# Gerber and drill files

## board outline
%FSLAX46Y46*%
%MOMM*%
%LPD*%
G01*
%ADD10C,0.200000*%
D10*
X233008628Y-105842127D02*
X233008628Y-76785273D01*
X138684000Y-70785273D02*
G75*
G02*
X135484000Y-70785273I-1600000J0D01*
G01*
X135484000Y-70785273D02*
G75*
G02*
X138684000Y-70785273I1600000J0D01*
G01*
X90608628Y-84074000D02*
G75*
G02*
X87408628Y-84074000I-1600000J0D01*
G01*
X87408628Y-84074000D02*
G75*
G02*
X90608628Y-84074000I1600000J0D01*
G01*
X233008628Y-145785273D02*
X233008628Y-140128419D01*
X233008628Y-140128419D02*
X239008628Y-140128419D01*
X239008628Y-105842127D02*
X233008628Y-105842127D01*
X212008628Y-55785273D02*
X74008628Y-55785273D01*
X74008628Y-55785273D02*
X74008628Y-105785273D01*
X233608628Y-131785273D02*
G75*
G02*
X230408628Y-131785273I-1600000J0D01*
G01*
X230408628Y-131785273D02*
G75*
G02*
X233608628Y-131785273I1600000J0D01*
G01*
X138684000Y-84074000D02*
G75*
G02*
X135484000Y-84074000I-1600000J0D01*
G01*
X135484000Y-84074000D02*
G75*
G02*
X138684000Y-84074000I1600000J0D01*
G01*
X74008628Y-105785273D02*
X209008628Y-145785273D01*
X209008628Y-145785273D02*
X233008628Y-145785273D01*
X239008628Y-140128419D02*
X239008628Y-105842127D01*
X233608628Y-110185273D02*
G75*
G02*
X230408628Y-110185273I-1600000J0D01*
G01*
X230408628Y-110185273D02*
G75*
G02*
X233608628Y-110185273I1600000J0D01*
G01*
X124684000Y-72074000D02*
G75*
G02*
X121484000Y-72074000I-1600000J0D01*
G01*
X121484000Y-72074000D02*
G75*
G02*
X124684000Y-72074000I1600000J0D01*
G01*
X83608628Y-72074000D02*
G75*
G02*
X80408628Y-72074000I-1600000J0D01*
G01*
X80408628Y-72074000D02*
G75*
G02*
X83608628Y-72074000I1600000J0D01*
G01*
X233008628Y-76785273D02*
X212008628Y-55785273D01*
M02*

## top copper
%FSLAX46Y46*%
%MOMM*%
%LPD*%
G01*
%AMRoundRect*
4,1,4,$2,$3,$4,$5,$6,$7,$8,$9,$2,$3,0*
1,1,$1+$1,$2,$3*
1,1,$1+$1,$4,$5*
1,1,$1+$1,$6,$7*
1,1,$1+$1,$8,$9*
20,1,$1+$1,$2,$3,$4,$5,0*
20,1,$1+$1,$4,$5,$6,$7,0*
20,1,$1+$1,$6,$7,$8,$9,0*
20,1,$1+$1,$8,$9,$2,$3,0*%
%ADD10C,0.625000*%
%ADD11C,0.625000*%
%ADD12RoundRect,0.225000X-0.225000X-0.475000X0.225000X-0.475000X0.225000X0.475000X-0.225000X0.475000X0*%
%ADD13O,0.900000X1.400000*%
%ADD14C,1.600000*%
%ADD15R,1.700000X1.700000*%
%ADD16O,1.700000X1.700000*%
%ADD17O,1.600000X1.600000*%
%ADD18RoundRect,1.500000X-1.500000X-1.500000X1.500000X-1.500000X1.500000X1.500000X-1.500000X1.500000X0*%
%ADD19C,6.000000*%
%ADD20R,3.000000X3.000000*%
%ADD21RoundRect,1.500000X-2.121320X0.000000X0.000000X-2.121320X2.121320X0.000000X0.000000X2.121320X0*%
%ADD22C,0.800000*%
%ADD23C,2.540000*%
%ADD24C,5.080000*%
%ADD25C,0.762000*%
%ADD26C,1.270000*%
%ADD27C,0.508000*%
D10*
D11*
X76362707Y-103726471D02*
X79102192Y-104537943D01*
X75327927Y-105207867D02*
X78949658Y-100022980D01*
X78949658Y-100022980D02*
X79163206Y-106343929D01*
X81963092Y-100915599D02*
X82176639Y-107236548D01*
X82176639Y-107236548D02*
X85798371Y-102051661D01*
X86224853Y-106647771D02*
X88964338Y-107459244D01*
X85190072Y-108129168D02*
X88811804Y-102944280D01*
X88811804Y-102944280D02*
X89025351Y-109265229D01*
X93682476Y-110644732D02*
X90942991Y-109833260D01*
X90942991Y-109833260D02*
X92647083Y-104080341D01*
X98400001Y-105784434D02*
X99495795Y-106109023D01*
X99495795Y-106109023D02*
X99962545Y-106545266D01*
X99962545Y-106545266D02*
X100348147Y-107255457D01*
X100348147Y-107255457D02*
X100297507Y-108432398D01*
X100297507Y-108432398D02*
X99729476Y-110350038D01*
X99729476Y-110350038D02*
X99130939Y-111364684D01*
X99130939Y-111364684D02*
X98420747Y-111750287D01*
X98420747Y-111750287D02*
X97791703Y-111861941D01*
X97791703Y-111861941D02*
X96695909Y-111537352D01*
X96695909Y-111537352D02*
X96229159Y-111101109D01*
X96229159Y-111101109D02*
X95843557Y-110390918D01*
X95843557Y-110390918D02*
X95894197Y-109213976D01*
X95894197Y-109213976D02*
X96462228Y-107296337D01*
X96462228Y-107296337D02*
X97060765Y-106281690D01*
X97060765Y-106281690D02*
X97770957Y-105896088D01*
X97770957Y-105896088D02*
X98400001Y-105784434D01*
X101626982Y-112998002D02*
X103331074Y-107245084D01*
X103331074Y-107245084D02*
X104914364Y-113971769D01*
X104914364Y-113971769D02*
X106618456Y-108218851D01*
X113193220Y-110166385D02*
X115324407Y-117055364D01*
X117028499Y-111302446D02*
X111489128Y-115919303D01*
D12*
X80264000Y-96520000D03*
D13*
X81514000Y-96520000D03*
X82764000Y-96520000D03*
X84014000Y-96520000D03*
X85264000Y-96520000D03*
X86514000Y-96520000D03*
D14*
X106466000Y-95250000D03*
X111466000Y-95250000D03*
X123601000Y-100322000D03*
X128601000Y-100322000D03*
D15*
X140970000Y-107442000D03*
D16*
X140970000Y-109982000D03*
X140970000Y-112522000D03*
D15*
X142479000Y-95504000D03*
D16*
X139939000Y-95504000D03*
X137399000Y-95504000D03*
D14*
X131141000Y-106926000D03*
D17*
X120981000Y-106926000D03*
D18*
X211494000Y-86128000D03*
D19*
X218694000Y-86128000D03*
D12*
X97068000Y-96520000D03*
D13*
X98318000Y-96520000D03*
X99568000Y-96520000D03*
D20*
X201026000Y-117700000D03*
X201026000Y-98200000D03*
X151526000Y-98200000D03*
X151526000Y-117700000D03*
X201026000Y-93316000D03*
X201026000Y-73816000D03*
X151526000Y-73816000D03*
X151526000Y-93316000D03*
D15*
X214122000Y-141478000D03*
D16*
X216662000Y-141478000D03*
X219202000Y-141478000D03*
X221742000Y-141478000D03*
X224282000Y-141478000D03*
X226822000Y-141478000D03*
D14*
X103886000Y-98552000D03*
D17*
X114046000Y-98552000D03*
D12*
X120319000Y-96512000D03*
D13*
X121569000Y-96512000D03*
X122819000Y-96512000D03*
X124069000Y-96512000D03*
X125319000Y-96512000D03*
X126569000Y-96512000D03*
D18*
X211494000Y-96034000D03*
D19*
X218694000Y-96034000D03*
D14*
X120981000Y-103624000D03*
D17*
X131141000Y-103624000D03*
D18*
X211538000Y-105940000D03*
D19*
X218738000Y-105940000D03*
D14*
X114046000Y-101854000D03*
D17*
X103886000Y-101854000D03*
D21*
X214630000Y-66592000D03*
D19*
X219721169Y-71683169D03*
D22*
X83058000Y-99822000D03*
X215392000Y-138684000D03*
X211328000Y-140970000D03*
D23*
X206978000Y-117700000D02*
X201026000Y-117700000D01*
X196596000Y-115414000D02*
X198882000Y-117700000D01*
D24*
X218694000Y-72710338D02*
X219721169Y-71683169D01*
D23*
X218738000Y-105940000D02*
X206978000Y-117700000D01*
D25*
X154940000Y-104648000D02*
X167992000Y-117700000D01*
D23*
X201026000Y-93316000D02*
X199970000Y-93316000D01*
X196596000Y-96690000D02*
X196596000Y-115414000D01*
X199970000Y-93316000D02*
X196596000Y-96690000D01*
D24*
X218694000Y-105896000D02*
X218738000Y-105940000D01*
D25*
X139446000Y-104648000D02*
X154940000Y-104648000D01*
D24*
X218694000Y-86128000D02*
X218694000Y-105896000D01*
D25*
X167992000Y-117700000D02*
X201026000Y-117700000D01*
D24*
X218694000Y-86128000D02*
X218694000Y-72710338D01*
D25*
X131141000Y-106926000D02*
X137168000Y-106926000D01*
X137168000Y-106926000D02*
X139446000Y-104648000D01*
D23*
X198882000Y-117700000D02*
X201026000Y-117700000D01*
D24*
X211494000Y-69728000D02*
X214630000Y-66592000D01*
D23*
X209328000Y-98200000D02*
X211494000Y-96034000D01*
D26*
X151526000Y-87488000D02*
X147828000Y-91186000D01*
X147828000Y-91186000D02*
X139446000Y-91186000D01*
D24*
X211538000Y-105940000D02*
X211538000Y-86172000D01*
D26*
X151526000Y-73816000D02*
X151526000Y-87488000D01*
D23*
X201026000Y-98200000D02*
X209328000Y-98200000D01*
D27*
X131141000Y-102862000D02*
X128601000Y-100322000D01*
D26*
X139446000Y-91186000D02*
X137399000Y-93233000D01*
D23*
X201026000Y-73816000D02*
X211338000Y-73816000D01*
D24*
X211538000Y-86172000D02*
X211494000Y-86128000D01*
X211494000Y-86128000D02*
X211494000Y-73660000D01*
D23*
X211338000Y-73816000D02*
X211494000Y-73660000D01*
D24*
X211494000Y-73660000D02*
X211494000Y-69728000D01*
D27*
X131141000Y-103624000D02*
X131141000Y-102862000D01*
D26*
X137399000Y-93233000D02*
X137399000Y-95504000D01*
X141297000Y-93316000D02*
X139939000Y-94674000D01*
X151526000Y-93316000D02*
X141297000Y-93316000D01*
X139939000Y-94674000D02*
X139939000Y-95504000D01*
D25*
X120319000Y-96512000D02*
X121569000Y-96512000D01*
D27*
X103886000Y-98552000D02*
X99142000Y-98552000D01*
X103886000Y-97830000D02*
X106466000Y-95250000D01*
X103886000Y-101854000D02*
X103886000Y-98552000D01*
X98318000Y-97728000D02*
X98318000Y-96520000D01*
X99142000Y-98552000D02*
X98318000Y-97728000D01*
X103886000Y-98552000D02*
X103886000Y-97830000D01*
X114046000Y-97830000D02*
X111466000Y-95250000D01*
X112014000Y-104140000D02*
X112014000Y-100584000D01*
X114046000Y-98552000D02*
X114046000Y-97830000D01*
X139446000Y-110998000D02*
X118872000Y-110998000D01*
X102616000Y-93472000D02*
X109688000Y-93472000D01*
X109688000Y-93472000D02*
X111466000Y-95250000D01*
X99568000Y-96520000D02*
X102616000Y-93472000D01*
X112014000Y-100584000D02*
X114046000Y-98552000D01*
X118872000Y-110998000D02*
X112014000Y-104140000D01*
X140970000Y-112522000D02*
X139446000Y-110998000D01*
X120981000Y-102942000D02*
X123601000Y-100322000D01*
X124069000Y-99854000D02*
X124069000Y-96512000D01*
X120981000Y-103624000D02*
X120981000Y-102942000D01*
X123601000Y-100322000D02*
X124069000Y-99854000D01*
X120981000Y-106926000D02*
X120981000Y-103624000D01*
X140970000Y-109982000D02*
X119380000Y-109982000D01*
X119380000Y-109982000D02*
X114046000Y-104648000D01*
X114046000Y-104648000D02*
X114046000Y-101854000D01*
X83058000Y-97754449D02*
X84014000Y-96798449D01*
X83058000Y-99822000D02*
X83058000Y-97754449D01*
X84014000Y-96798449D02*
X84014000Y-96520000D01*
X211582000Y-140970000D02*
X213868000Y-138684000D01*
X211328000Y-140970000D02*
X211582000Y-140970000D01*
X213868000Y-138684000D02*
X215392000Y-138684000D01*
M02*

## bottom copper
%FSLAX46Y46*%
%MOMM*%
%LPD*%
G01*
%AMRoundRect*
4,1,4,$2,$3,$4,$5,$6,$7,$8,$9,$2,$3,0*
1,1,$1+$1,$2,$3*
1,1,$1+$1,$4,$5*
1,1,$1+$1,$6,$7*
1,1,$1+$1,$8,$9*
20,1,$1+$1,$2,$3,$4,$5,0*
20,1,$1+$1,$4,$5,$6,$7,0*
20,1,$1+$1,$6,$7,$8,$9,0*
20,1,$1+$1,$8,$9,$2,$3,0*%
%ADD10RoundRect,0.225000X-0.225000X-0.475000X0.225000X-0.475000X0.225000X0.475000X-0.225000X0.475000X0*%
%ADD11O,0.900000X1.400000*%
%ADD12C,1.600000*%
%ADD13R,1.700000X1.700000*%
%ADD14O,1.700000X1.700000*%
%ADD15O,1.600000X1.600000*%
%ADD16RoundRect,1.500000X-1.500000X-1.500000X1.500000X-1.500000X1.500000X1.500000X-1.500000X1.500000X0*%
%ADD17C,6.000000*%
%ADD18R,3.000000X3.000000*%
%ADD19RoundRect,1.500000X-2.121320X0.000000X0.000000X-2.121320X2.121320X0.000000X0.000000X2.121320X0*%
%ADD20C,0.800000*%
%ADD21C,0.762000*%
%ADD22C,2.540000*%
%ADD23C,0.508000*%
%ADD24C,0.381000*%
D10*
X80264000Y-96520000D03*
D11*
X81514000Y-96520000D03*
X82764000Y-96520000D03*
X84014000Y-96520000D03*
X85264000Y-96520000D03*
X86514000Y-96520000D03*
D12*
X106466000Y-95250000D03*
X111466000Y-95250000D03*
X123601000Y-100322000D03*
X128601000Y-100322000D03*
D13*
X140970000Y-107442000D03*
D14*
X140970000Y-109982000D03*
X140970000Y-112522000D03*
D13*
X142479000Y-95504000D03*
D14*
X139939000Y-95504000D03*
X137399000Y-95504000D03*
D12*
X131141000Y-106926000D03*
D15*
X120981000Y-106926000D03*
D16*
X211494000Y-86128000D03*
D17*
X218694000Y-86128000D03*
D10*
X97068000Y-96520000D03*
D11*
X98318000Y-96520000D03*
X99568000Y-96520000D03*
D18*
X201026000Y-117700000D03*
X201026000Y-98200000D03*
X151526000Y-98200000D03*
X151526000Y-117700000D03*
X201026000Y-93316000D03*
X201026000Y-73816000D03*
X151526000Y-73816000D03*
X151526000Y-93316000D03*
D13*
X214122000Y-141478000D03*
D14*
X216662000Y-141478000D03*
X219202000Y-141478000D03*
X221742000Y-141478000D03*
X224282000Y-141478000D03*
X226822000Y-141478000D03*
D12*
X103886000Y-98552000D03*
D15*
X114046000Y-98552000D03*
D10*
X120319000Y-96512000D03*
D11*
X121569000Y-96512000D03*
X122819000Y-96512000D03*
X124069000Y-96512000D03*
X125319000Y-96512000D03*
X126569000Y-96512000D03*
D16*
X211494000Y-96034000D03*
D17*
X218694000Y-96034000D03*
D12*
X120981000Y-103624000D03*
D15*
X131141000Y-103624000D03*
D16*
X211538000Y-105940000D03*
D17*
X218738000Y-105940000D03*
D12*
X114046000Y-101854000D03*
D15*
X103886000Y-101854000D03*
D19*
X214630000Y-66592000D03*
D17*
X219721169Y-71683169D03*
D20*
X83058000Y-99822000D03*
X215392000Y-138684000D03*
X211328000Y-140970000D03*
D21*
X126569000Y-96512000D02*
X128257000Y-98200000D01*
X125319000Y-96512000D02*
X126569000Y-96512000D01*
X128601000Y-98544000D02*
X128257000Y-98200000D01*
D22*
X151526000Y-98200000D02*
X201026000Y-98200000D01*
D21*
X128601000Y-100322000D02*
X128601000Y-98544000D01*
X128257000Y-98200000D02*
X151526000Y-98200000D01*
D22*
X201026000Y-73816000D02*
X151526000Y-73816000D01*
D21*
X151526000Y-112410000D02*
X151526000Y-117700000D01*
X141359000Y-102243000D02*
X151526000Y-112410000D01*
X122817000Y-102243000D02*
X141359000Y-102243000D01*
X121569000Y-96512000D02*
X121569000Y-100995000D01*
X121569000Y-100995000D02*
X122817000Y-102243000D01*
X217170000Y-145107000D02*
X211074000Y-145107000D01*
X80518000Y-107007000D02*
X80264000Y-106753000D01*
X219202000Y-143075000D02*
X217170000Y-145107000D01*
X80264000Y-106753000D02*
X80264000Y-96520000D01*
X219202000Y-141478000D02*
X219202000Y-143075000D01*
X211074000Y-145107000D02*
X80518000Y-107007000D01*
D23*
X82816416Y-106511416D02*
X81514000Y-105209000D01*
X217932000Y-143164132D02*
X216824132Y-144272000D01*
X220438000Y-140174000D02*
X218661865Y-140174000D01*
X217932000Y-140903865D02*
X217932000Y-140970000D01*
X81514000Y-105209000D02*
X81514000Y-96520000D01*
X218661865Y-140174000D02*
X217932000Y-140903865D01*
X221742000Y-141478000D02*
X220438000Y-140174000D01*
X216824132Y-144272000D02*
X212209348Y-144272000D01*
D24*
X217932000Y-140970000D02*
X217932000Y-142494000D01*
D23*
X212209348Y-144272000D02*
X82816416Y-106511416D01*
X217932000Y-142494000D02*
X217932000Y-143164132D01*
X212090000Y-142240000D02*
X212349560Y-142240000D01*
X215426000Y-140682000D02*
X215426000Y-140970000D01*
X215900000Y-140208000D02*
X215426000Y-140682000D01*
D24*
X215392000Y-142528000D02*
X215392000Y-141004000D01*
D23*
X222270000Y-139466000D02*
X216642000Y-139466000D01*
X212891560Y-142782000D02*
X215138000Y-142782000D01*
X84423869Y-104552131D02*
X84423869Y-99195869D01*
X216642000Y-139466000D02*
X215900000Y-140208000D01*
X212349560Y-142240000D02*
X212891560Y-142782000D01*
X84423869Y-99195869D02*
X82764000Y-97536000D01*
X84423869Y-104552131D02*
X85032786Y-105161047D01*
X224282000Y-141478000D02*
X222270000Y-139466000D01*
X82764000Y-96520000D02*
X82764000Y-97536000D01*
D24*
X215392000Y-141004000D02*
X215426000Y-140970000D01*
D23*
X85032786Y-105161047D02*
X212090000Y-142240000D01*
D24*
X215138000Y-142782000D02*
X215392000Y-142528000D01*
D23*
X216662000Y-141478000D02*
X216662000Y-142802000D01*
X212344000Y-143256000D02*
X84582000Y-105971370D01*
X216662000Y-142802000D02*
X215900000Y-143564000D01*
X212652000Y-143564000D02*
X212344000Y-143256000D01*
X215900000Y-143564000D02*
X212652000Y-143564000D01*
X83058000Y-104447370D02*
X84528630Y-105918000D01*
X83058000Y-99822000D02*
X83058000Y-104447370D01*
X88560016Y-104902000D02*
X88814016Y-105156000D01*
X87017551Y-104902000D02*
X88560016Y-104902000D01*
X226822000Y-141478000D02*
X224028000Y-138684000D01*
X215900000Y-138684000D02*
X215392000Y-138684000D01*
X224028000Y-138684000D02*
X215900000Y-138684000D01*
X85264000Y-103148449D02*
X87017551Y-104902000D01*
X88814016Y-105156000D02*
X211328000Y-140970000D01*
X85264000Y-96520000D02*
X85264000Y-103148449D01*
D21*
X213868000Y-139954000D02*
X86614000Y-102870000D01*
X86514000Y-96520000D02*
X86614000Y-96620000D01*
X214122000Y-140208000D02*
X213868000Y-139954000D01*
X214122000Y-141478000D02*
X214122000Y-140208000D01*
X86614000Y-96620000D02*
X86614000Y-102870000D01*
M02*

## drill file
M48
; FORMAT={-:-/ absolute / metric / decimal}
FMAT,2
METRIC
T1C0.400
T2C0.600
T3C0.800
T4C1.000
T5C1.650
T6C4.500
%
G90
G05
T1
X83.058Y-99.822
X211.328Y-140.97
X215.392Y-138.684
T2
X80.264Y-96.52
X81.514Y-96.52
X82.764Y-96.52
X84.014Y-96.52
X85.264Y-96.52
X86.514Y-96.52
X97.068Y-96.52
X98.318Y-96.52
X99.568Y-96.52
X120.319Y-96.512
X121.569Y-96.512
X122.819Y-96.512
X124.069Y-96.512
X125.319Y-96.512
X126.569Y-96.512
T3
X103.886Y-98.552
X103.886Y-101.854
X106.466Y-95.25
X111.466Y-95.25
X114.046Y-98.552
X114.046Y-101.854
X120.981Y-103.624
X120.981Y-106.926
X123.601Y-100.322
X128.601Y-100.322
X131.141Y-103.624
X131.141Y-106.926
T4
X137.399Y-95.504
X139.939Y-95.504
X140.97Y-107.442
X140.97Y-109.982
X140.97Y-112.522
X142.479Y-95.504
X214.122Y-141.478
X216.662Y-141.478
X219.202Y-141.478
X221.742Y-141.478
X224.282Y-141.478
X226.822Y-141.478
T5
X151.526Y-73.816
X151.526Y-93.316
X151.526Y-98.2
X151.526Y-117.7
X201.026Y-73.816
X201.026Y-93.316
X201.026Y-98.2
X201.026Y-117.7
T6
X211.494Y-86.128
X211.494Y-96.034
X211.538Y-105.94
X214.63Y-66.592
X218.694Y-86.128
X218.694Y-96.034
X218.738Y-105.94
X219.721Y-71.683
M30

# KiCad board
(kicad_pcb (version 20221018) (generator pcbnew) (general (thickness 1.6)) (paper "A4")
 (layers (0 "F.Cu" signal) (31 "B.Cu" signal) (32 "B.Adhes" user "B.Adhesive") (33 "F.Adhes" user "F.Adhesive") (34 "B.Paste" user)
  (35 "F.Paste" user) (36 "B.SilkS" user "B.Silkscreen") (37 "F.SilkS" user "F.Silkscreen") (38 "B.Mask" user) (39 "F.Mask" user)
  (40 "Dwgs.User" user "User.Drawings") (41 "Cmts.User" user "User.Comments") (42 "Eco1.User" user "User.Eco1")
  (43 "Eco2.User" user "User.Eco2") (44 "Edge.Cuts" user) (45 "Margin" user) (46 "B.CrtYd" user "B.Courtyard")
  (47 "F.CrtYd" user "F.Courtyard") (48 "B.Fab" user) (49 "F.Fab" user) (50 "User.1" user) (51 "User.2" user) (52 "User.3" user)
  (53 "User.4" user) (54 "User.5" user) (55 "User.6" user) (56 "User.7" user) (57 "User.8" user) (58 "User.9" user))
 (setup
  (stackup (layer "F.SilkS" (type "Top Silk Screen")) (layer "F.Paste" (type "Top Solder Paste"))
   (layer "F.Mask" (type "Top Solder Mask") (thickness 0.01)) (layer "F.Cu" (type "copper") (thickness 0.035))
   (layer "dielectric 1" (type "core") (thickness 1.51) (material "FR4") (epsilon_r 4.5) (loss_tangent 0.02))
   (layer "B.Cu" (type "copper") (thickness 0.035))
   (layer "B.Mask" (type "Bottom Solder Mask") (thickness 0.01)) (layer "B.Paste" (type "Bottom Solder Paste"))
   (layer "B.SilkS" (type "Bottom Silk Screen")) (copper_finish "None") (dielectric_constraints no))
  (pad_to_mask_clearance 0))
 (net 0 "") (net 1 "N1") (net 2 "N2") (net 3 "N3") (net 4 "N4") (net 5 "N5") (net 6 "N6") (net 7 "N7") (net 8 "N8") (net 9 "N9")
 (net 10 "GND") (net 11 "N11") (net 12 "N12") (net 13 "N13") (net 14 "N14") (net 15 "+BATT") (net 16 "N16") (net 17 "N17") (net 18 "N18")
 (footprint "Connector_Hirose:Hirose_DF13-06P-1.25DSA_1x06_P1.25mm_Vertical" (layer "F.Cu") (at 80.264 96.52)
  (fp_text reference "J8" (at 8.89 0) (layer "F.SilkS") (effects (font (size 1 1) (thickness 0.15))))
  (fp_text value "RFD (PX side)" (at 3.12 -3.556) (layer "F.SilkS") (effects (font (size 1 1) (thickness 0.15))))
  (pad "1" thru_hole roundrect (at 0 0) (size 0.9 1.4) (drill 0.6) (layers "*.Cu" "*.Mask") (roundrect_rratio 0.25) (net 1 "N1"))
  (pad "2" thru_hole oval (at 1.25 0) (size 0.9 1.4) (drill 0.6) (layers "*.Cu" "*.Mask") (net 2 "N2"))
  (pad "3" thru_hole oval (at 2.5 0) (size 0.9 1.4) (drill 0.6) (layers "*.Cu" "*.Mask") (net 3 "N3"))
  (pad "4" thru_hole oval (at 3.75 0) (size 0.9 1.4) (drill 0.6) (layers "*.Cu" "*.Mask") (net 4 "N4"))
  (pad "5" thru_hole oval (at 5 0) (size 0.9 1.4) (drill 0.6) (layers "*.Cu" "*.Mask") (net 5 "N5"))
  (pad "6" thru_hole oval (at 6.25 0) (size 0.9 1.4) (drill 0.6) (layers "*.Cu" "*.Mask") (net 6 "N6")))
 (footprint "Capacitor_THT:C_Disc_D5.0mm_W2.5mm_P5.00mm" (layer "F.Cu") (at 106.466 95.25)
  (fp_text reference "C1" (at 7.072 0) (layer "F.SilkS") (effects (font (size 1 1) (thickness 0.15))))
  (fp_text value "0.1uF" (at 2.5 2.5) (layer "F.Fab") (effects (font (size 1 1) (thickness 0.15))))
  (pad "1" thru_hole circle (at 0 0) (size 1.6 1.6) (drill 0.8) (layers "*.Cu" "*.Mask") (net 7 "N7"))
  (pad "2" thru_hole circle (at 5 0) (size 1.6 1.6) (drill 0.8) (layers "*.Cu" "*.Mask") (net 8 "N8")))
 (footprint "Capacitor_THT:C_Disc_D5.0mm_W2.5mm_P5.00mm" (layer "F.Cu") (at 123.601 100.322)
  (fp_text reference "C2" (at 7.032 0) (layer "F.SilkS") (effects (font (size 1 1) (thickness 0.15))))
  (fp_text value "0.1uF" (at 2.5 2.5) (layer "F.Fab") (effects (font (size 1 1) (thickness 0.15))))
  (pad "1" thru_hole circle (at 0 0) (size 1.6 1.6) (drill 0.8) (layers "*.Cu" "*.Mask") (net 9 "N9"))
  (pad "2" thru_hole circle (at 5 0) (size 1.6 1.6) (drill 0.8) (layers "*.Cu" "*.Mask") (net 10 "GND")))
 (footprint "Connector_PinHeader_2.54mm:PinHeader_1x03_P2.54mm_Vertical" (layer "F.Cu") (at 140.97 107.442)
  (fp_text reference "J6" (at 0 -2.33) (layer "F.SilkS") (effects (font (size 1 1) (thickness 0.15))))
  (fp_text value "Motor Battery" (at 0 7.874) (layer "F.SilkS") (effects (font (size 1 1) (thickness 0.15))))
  (pad "1" thru_hole rect (at 0 0) (size 1.7 1.7) (drill 1) (layers "*.Cu" "*.Mask") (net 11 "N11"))
  (pad "2" thru_hole oval (at 0 2.54) (size 1.7 1.7) (drill 1) (layers "*.Cu" "*.Mask") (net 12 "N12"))
  (pad "3" thru_hole oval (at 0 5.08) (size 1.7 1.7) (drill 1) (layers "*.Cu" "*.Mask") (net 8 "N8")))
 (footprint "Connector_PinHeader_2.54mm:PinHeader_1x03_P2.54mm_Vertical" (layer "F.Cu") (at 142.479 95.504 -90)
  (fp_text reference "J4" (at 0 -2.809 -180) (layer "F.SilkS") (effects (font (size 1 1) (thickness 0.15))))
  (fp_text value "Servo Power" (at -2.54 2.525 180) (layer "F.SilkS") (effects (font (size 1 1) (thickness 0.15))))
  (pad "1" thru_hole rect (at 0 0 270) (size 1.7 1.7) (drill 1) (layers "*.Cu" "*.Mask") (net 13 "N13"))
  (pad "2" thru_hole oval (at 0 2.54 270) (size 1.7 1.7) (drill 1) (layers "*.Cu" "*.Mask") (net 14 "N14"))
  (pad "3" thru_hole oval (at 0 5.08 270) (size 1.7 1.7) (drill 1) (layers "*.Cu" "*.Mask") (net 10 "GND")))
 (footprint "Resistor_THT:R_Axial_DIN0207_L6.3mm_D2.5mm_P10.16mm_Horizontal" (layer "F.Cu") (at 131.141 106.926 180)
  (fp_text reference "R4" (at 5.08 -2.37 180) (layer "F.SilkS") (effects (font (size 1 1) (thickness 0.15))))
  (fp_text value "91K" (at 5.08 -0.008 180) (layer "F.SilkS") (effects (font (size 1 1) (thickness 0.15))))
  (pad "1" thru_hole circle (at 0 0 180) (size 1.6 1.6) (drill 0.8) (layers "*.Cu" "*.Mask") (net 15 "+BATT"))
  (pad "2" thru_hole oval (at 10.16 0 180) (size 1.6 1.6) (drill 0.8) (layers "*.Cu" "*.Mask") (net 9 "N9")))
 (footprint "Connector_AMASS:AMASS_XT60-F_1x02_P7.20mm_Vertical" (layer "F.Cu") (at 211.494 86.128)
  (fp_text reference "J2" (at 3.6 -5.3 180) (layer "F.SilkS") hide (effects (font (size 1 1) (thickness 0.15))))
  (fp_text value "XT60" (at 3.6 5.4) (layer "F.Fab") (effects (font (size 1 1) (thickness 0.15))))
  (pad "1" thru_hole roundrect (at 0 0) (size 6 6) (drill 4.5) (layers "*.Cu" "*.Mask") (roundrect_rratio 0.25) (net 10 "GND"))
  (pad "2" thru_hole circle (at 7.2 0) (size 6 6) (drill 4.5) (layers "*.Cu" "*.Mask") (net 15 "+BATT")))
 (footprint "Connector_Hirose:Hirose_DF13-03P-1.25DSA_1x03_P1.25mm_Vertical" (layer "F.Cu") (at 97.068 96.52)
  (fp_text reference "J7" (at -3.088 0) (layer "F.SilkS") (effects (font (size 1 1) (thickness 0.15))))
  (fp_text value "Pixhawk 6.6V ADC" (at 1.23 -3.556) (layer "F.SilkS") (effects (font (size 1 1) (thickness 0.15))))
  (pad "1" thru_hole roundrect (at 0 0) (size 0.9 1.4) (drill 0.6) (layers "*.Cu" "*.Mask") (roundrect_rratio 0.25) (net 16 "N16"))
  (pad "2" thru_hole oval (at 1.25 0) (size 0.9 1.4) (drill 0.6) (layers "*.Cu" "*.Mask") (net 7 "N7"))
  (pad "3" thru_hole oval (at 2.5 0) (size 0.9 1.4) (drill 0.6) (layers "*.Cu" "*.Mask") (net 8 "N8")))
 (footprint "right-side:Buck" (layer "F.Cu") (at 176.276 107.95 180)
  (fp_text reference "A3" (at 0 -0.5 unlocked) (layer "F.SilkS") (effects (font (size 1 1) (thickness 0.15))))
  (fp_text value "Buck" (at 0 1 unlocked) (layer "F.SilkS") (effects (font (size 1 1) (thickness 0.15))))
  (pad "1" thru_hole rect (at -24.75 -9.75 180) (size 3 3) (drill 1.65) (layers "*.Cu" "*.Mask") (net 15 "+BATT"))
  (pad "2" thru_hole rect (at -24.75 9.75 180) (size 3 3) (drill 1.65) (layers "*.Cu" "*.Mask") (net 10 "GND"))
  (pad "3" thru_hole rect (at 24.75 9.75 180) (size 3 3) (drill 1.65) (layers "*.Cu" "*.Mask") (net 10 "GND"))
  (pad "4" thru_hole rect (at 24.75 -9.75 180) (size 3 3) (drill 1.65) (layers "*.Cu" "*.Mask") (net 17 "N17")))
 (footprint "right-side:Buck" (layer "F.Cu") (at 176.276 83.566 180)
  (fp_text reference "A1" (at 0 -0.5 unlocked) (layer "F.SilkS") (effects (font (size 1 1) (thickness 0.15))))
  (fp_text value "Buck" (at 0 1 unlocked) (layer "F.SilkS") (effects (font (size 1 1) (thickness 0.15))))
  (pad "1" thru_hole rect (at -24.75 -9.75 180) (size 3 3) (drill 1.65) (layers "*.Cu" "*.Mask") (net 15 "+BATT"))
  (pad "2" thru_hole rect (at -24.75 9.75 180) (size 3 3) (drill 1.65) (layers "*.Cu" "*.Mask") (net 10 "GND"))
  (pad "3" thru_hole rect (at 24.75 9.75 180) (size 3 3) (drill 1.65) (layers "*.Cu" "*.Mask") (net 10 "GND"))
  (pad "4" thru_hole rect (at 24.75 -9.75 180) (size 3 3) (drill 1.65) (layers "*.Cu" "*.Mask") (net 14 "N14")))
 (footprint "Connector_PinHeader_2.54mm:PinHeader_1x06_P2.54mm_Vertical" (layer "F.Cu") (at 214.122 141.478 90)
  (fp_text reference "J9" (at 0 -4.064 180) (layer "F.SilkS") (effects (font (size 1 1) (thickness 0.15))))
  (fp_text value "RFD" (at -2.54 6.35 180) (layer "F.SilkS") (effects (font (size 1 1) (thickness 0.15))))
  (pad "1" thru_hole rect (at 0 0 90) (size 1.7 1.7) (drill 1) (layers "*.Cu" "*.Mask") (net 6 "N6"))
  (pad "2" thru_hole oval (at 0 2.54 90) (size 1.7 1.7) (drill 1) (layers "*.Cu" "*.Mask") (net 4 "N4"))
  (pad "3" thru_hole oval (at 0 5.08 90) (size 1.7 1.7) (drill 1) (layers "*.Cu" "*.Mask") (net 1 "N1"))
  (pad "4" thru_hole oval (at 0 7.62 90) (size 1.7 1.7) (drill 1) (layers "*.Cu" "*.Mask") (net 2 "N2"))
  (pad "5" thru_hole oval (at 0 10.16 90) (size 1.7 1.7) (drill 1) (layers "*.Cu" "*.Mask") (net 3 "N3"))
  (pad "6" thru_hole oval (at 0 12.7 90) (size 1.7 1.7) (drill 1) (layers "*.Cu" "*.Mask") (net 5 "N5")))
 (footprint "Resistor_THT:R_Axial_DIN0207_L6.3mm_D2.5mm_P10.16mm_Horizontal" (layer "F.Cu") (at 103.886 98.552)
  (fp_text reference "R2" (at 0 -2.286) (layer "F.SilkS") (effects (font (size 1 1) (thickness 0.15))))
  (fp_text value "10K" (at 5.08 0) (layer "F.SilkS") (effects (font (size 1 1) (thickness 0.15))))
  (pad "1" thru_hole circle (at 0 0) (size 1.6 1.6) (drill 0.8) (layers "*.Cu" "*.Mask") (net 7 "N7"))
  (pad "2" thru_hole oval (at 10.16 0) (size 1.6 1.6) (drill 0.8) (layers "*.Cu" "*.Mask") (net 8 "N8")))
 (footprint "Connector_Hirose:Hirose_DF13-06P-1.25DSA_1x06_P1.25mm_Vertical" (layer "F.Cu") (at 120.319 96.512)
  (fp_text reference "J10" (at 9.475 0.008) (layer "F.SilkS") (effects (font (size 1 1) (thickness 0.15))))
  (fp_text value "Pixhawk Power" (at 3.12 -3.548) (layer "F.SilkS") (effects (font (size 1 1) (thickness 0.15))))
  (pad "1" thru_hole roundrect (at 0 0) (size 0.9 1.4) (drill 0.6) (layers "*.Cu" "*.Mask") (roundrect_rratio 0.25) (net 17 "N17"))
  (pad "2" thru_hole oval (at 1.25 0) (size 0.9 1.4) (drill 0.6) (layers "*.Cu" "*.Mask") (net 17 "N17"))
  (pad "3" thru_hole oval (at 2.5 0) (size 0.9 1.4) (drill 0.6) (layers "*.Cu" "*.Mask") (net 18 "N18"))
  (pad "4" thru_hole oval (at 3.75 0) (size 0.9 1.4) (drill 0.6) (layers "*.Cu" "*.Mask") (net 9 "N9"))
  (pad "5" thru_hole oval (at 5 0) (size 0.9 1.4) (drill 0.6) (layers "*.Cu" "*.Mask") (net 10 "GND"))
  (pad "6" thru_hole oval (at 6.25 0) (size 0.9 1.4) (drill 0.6) (layers "*.Cu" "*.Mask") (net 10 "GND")))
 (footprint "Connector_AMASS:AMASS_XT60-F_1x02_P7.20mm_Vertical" (layer "F.Cu") (at 211.494 96.034)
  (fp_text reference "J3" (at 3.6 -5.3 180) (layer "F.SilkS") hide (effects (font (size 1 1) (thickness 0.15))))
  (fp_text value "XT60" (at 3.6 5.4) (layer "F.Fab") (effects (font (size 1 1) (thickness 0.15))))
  (pad "1" thru_hole roundrect (at 0 0) (size 6 6) (drill 4.5) (layers "*.Cu" "*.Mask") (roundrect_rratio 0.25) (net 10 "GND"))
  (pad "2" thru_hole circle (at 7.2 0) (size 6 6) (drill 4.5) (layers "*.Cu" "*.Mask") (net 15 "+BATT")))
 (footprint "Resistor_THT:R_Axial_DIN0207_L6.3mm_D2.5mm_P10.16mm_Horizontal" (layer "F.Cu") (at 120.981 103.624)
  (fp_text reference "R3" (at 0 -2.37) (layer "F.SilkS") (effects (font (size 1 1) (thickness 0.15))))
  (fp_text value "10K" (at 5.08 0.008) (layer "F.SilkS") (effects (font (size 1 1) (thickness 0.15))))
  (pad "1" thru_hole circle (at 0 0) (size 1.6 1.6) (drill 0.8) (layers "*.Cu" "*.Mask") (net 9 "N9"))
  (pad "2" thru_hole oval (at 10.16 0) (size 1.6 1.6) (drill 0.8) (layers "*.Cu" "*.Mask") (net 10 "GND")))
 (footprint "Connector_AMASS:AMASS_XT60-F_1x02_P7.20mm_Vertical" (layer "F.Cu") (at 211.538 105.94)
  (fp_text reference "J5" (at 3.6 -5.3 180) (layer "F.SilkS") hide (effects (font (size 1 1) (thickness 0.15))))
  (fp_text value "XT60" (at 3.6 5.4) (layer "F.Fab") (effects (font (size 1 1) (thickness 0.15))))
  (pad "1" thru_hole roundrect (at 0 0) (size 6 6) (drill 4.5) (layers "*.Cu" "*.Mask") (roundrect_rratio 0.25) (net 10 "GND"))
  (pad "2" thru_hole circle (at 7.2 0) (size 6 6) (drill 4.5) (layers "*.Cu" "*.Mask") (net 15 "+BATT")))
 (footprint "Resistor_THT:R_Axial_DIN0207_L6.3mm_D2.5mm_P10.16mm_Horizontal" (layer "F.Cu") (at 114.046 101.854 180)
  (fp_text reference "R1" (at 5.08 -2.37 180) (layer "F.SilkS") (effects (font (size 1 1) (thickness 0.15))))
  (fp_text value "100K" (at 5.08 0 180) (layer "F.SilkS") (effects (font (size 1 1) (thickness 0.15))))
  (pad "1" thru_hole circle (at 0 0 180) (size 1.6 1.6) (drill 0.8) (layers "*.Cu" "*.Mask") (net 12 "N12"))
  (pad "2" thru_hole oval (at 10.16 0 180) (size 1.6 1.6) (drill 0.8) (layers "*.Cu" "*.Mask") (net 7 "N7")))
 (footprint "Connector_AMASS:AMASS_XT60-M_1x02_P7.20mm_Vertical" (layer "B.Cu") (at 214.63 66.592 -45)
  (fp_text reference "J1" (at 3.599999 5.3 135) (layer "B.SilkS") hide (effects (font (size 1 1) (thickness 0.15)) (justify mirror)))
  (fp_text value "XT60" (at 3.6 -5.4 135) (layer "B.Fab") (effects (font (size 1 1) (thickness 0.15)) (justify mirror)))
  (pad "1" thru_hole roundrect (at 0 0 315) (size 6 6) (drill 4.5) (layers "*.Cu" "*.Mask") (roundrect_rratio 0.25) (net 10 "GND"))
  (pad "2" thru_hole circle (at 7.2 0 315) (size 6 6) (drill 4.5) (layers "*.Cu" "*.Mask") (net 15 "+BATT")))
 (gr_line (start 233.008628 105.842127) (end 233.008628 76.785273) (stroke (width 0.2) (type solid)) (layer "Edge.Cuts"))
 (gr_circle (center 137.084 70.785273) (end 138.684 70.785273) (stroke (width 0.2) (type solid)) (fill none) (layer "Edge.Cuts"))
 (gr_circle (center 89.008628 84.074) (end 90.608628 84.074) (stroke (width 0.2) (type solid)) (fill none) (layer "Edge.Cuts"))
 (gr_line (start 233.008628 145.785273) (end 233.008628 140.128419) (stroke (width 0.2) (type solid)) (layer "Edge.Cuts"))
 (gr_line (start 233.008628 140.128419) (end 239.008628 140.128419) (stroke (width 0.2) (type solid)) (layer "Edge.Cuts"))
 (gr_line (start 239.008628 105.842127) (end 233.008628 105.842127) (stroke (width 0.2) (type solid)) (layer "Edge.Cuts"))
 (gr_line (start 212.008628 55.785273) (end 74.008628 55.785273) (stroke (width 0.2) (type solid)) (layer "Edge.Cuts"))
 (gr_line (start 74.008628 55.785273) (end 74.008628 105.785273) (stroke (width 0.2) (type solid)) (layer "Edge.Cuts"))
 (gr_circle (center 232.008628 131.785273) (end 233.608628 131.785273) (stroke (width 0.2) (type solid)) (fill none) (layer "Edge.Cuts"))
 (gr_circle (center 137.084 84.074) (end 138.684 84.074) (stroke (width 0.2) (type solid)) (fill none) (layer "Edge.Cuts"))
 (gr_line (start 74.008628 105.785273) (end 209.008628 145.785273) (stroke (width 0.2) (type solid)) (layer "Edge.Cuts"))
 (gr_line (start 209.008628 145.785273) (end 233.008628 145.785273) (stroke (width 0.2) (type solid)) (layer "Edge.Cuts"))
 (gr_line (start 239.008628 140.128419) (end 239.008628 105.842127) (stroke (width 0.2) (type solid)) (layer "Edge.Cuts"))
 (gr_circle (center 232.008628 110.185273) (end 233.608628 110.185273) (stroke (width 0.2) (type solid)) (fill none) (layer "Edge.Cuts"))
 (gr_circle (center 123.084 72.074) (end 124.684 72.074) (stroke (width 0.2) (type solid)) (fill none) (layer "Edge.Cuts"))
 (gr_circle (center 82.008628 72.074) (end 83.608628 72.074) (stroke (width 0.2) (type solid)) (fill none) (layer "Edge.Cuts"))
 (gr_line (start 233.008628 76.785273) (end 212.008628 55.785273) (stroke (width 0.2) (type solid)) (layer "Edge.Cuts"))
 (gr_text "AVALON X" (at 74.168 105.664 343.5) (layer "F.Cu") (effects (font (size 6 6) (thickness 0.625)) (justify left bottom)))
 (segment (start 206.978 117.7) (end 201.026 117.7) (width 2.54) (layer "F.Cu") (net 15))
 (segment (start 196.596 115.414) (end 198.882 117.7) (width 2.54) (layer "F.Cu") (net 15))
 (segment (start 218.694 72.710338) (end 219.721169 71.683169) (width 5.08) (layer "F.Cu") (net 15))
 (segment (start 218.738 105.94) (end 206.978 117.7) (width 2.54) (layer "F.Cu") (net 15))
 (segment (start 154.94 104.648) (end 167.992 117.7) (width 0.762) (layer "F.Cu") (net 15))
 (segment (start 201.026 93.316) (end 199.97 93.316) (width 2.54) (layer "F.Cu") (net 15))
 (segment (start 196.596 96.69) (end 196.596 115.414) (width 2.54) (layer "F.Cu") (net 15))
 (segment (start 199.97 93.316) (end 196.596 96.69) (width 2.54) (layer "F.Cu") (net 15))
 (segment (start 218.694 105.896) (end 218.738 105.94) (width 5.08) (layer "F.Cu") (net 15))
 (segment (start 139.446 104.648) (end 154.94 104.648) (width 0.762) (layer "F.Cu") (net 15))
 (segment (start 218.694 86.128) (end 218.694 105.896) (width 5.08) (layer "F.Cu") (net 15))
 (segment (start 167.992 117.7) (end 201.026 117.7) (width 0.762) (layer "F.Cu") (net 15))
 (segment (start 218.694 86.128) (end 218.694 72.710338) (width 5.08) (layer "F.Cu") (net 15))
 (segment (start 131.141 106.926) (end 137.168 106.926) (width 0.762) (layer "F.Cu") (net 15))
 (segment (start 137.168 106.926) (end 139.446 104.648) (width 0.762) (layer "F.Cu") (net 15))
 (segment (start 198.882 117.7) (end 201.026 117.7) (width 2.54) (layer "F.Cu") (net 15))
 (segment (start 211.494 69.728) (end 214.63 66.592) (width 5.08) (layer "F.Cu") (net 10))
 (segment (start 209.328 98.2) (end 211.494 96.034) (width 2.54) (layer "F.Cu") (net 10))
 (segment (start 151.526 87.488) (end 147.828 91.186) (width 1.27) (layer "F.Cu") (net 10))
 (segment (start 147.828 91.186) (end 139.446 91.186) (width 1.27) (layer "F.Cu") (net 10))
 (segment (start 211.538 105.94) (end 211.538 86.172) (width 5.08) (layer "F.Cu") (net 10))
 (segment (start 151.526 73.816) (end 151.526 87.488) (width 1.27) (layer "F.Cu") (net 10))
 (segment (start 201.026 98.2) (end 209.328 98.2) (width 2.54) (layer "F.Cu") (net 10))
 (segment (start 131.141 102.862) (end 128.601 100.322) (width 0.508) (layer "F.Cu") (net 10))
 (segment (start 139.446 91.186) (end 137.399 93.233) (width 1.27) (layer "F.Cu") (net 10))
 (segment (start 201.026 73.816) (end 211.338 73.816) (width 2.54) (layer "F.Cu") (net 10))
 (segment (start 211.538 86.172) (end 211.494 86.128) (width 5.08) (layer "F.Cu") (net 10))
 (segment (start 211.494 86.128) (end 211.494 73.66) (width 5.08) (layer "F.Cu") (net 10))
 (segment (start 211.338 73.816) (end 211.494 73.66) (width 2.54) (layer "F.Cu") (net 10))
 (segment (start 211.494 73.66) (end 211.494 69.728) (width 5.08) (layer "F.Cu") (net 10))
 (segment (start 131.141 103.624) (end 131.141 102.862) (width 0.508) (layer "F.Cu") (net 10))
 (segment (start 137.399 93.233) (end 137.399 95.504) (width 1.27) (layer "F.Cu") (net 10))
 (segment (start 126.569 96.512) (end 128.257 98.2) (width 0.762) (layer "B.Cu") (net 10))
 (segment (start 125.319 96.512) (end 126.569 96.512) (width 0.762) (layer "B.Cu") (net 10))
 (segment (start 128.601 98.544) (end 128.257 98.2) (width 0.762) (layer "B.Cu") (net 10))
 (segment (start 151.526 98.2) (end 201.026 98.2) (width 2.54) (layer "B.Cu") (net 10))
 (segment (start 128.601 100.322) (end 128.601 98.544) (width 0.762) (layer "B.Cu") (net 10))
 (segment (start 128.257 98.2) (end 151.526 98.2) (width 0.762) (layer "B.Cu") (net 10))
 (segment (start 201.026 73.816) (end 151.526 73.816) (width 2.54) (layer "B.Cu") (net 10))
 (segment (start 141.297 93.316) (end 139.939 94.674) (width 1.27) (layer "F.Cu") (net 14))
 (segment (start 151.526 93.316) (end 141.297 93.316) (width 1.27) (layer "F.Cu") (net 14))
 (segment (start 139.939 94.674) (end 139.939 95.504) (width 1.27) (layer "F.Cu") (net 14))
 (segment (start 120.319 96.512) (end 121.569 96.512) (width 0.762) (layer "F.Cu") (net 17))
 (segment (start 151.526 112.41) (end 151.526 117.7) (width 0.762) (layer "B.Cu") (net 17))
 (segment (start 141.359 102.243) (end 151.526 112.41) (width 0.762) (layer "B.Cu") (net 17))
 (segment (start 122.817 102.243) (end 141.359 102.243) (width 0.762) (layer "B.Cu") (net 17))
 (segment (start 121.569 96.512) (end 121.569 100.995) (width 0.762) (layer "B.Cu") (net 17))
 (segment (start 121.569 100.995) (end 122.817 102.243) (width 0.762) (layer "B.Cu") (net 17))
 (segment (start 103.886 98.552) (end 99.142 98.552) (width 0.508) (layer "F.Cu") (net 7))
 (segment (start 103.886 97.83) (end 106.466 95.25) (width 0.508) (layer "F.Cu") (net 7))
 (segment (start 103.886 101.854) (end 103.886 98.552) (width 0.508) (layer "F.Cu") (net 7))
 (segment (start 98.318 97.728) (end 98.318 96.52) (width 0.508) (layer "F.Cu") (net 7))
 (segment (start 99.142 98.552) (end 98.318 97.728) (width 0.508) (layer "F.Cu") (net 7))
 (segment (start 103.886 98.552) (end 103.886 97.83) (width 0.508) (layer "F.Cu") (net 7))
 (segment (start 114.046 97.83) (end 111.466 95.25) (width 0.508) (layer "F.Cu") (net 8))
 (segment (start 112.014 104.14) (end 112.014 100.584) (width 0.508) (layer "F.Cu") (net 8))
 (segment (start 114.046 98.552) (end 114.046 97.83) (width 0.508) (layer "F.Cu") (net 8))
 (segment (start 139.446 110.998) (end 118.872 110.998) (width 0.508) (layer "F.Cu") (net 8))
 (segment (start 102.616 93.472) (end 109.688 93.472) (width 0.508) (layer "F.Cu") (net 8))
 (segment (start 109.688 93.472) (end 111.466 95.25) (width 0.508) (layer "F.Cu") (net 8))
 (segment (start 99.568 96.52) (end 102.616 93.472) (width 0.508) (layer "F.Cu") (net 8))
 (segment (start 112.014 100.584) (end 114.046 98.552) (width 0.508) (layer "F.Cu") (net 8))
 (segment (start 118.872 110.998) (end 112.014 104.14) (width 0.508) (layer "F.Cu") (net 8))
 (segment (start 140.97 112.522) (end 139.446 110.998) (width 0.508) (layer "F.Cu") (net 8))
 (segment (start 120.981 102.942) (end 123.601 100.322) (width 0.508) (layer "F.Cu") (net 9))
 (segment (start 124.069 99.854) (end 124.069 96.512) (width 0.508) (layer "F.Cu") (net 9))
 (segment (start 120.981 103.624) (end 120.981 102.942) (width 0.508) (layer "F.Cu") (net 9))
 (segment (start 123.601 100.322) (end 124.069 99.854) (width 0.508) (layer "F.Cu") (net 9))
 (segment (start 120.981 106.926) (end 120.981 103.624) (width 0.508) (layer "F.Cu") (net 9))
 (segment (start 140.97 109.982) (end 119.38 109.982) (width 0.508) (layer "F.Cu") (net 12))
 (segment (start 119.38 109.982) (end 114.046 104.648) (width 0.508) (layer "F.Cu") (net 12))
 (segment (start 114.046 104.648) (end 114.046 101.854) (width 0.508) (layer "F.Cu") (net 12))
 (segment (start 217.17 145.107) (end 211.074 145.107) (width 0.762) (layer "B.Cu") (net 1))
 (segment (start 80.518 107.007) (end 80.264 106.753) (width 0.762) (layer "B.Cu") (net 1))
 (segment (start 219.202 143.075) (end 217.17 145.107) (width 0.762) (layer "B.Cu") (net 1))
 (segment (start 80.264 106.753) (end 80.264 96.52) (width 0.762) (layer "B.Cu") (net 1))
 (segment (start 219.202 141.478) (end 219.202 143.075) (width 0.762) (layer "B.Cu") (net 1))
 (segment (start 211.074 145.107) (end 80.518 107.007) (width 0.762) (layer "B.Cu") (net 1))
 (segment (start 82.816416 106.511416) (end 81.514 105.209) (width 0.508) (layer "B.Cu") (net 2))
 (segment (start 217.932 143.164132) (end 216.824132 144.272) (width 0.508) (layer "B.Cu") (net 2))
 (segment (start 220.438 140.174) (end 218.661865 140.174) (width 0.508) (layer "B.Cu") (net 2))
 (segment (start 217.932 140.903865) (end 217.932 140.97) (width 0.508) (layer "B.Cu") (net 2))
 (segment (start 81.514 105.209) (end 81.514 96.52) (width 0.508) (layer "B.Cu") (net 2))
 (segment (start 218.661865 140.174) (end 217.932 140.903865) (width 0.508) (layer "B.Cu") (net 2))
 (segment (start 221.742 141.478) (end 220.438 140.174) (width 0.508) (layer "B.Cu") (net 2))
 (segment (start 216.824132 144.272) (end 212.209348 144.272) (width 0.508) (layer "B.Cu") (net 2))
 (segment (start 217.932 140.97) (end 217.932 142.494) (width 0.381) (layer "B.Cu") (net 2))
 (segment (start 212.209348 144.272) (end 82.816416 106.511416) (width 0.508) (layer "B.Cu") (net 2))
 (segment (start 217.932 142.494) (end 217.932 143.164132) (width 0.508) (layer "B.Cu") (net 2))
 (segment (start 212.09 142.24) (end 212.34956 142.24) (width 0.508) (layer "B.Cu") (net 3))
 (segment (start 215.426 140.682) (end 215.426 140.97) (width 0.508) (layer "B.Cu") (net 3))
 (segment (start 215.9 140.208) (end 215.426 140.682) (width 0.508) (layer "B.Cu") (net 3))
 (segment (start 215.392 142.528) (end 215.392 141.004) (width 0.381) (layer "B.Cu") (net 3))
 (segment (start 222.27 139.466) (end 216.642 139.466) (width 0.508) (layer "B.Cu") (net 3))
 (segment (start 212.89156 142.782) (end 215.138 142.782) (width 0.508) (layer "B.Cu") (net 3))
 (segment (start 84.423869 104.552131) (end 84.423869 99.195869) (width 0.508) (layer "B.Cu") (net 3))
 (segment (start 216.642 139.466) (end 215.9 140.208) (width 0.508) (layer "B.Cu") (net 3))
 (segment (start 212.34956 142.24) (end 212.89156 142.782) (width 0.508) (layer "B.Cu") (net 3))
 (segment (start 84.423869 99.195869) (end 82.764 97.536) (width 0.508) (layer "B.Cu") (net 3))
 (segment (start 84.423869 104.552131) (end 85.032786 105.161047) (width 0.508) (layer "B.Cu") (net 3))
 (segment (start 224.282 141.478) (end 222.27 139.466) (width 0.508) (layer "B.Cu") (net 3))
 (segment (start 82.764 96.52) (end 82.764 97.536) (width 0.508) (layer "B.Cu") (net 3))
 (segment (start 215.392 141.004) (end 215.426 140.97) (width 0.381) (layer "B.Cu") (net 3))
 (segment (start 85.032786 105.161047) (end 212.09 142.24) (width 0.508) (layer "B.Cu") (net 3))
 (segment (start 215.138 142.782) (end 215.392 142.528) (width 0.381) (layer "B.Cu") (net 3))
 (segment (start 83.058 97.754449) (end 84.014 96.798449) (width 0.508) (layer "F.Cu") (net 4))
 (segment (start 83.058 99.822) (end 83.058 97.754449) (width 0.508) (layer "F.Cu") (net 4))
 (segment (start 84.014 96.798449) (end 84.014 96.52) (width 0.508) (layer "F.Cu") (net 4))
 (via (at 83.058 99.822) (size 0.8) (drill 0.4) (layers "F.Cu" "B.Cu") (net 4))
 (segment (start 216.662 141.478) (end 216.662 142.802) (width 0.508) (layer "B.Cu") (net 4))
 (segment (start 212.344 143.256) (end 84.582 105.97137) (width 0.508) (layer "B.Cu") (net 4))
 (segment (start 216.662 142.802) (end 215.9 143.564) (width 0.508) (layer "B.Cu") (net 4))
 (segment (start 212.652 143.564) (end 212.344 143.256) (width 0.508) (layer "B.Cu") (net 4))
 (segment (start 215.9 143.564) (end 212.652 143.564) (width 0.508) (layer "B.Cu") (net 4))
 (segment (start 83.058 104.44737) (end 84.52863 105.918) (width 0.508) (layer "B.Cu") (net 4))
 (segment (start 83.058 99.822) (end 83.058 104.44737) (width 0.508) (layer "B.Cu") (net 4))
 (segment (start 211.582 140.97) (end 213.868 138.684) (width 0.508) (layer "F.Cu") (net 5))
 (segment (start 211.328 140.97) (end 211.582 140.97) (width 0.508) (layer "F.Cu") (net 5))
 (segment (start 213.868 138.684) (end 215.392 138.684) (width 0.508) (layer "F.Cu") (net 5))
 (via (at 215.392 138.684) (size 0.8) (drill 0.4) (layers "F.Cu" "B.Cu") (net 5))
 (via (at 211.328 140.97) (size 0.8) (drill 0.4) (layers "F.Cu" "B.Cu") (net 5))
 (segment (start 88.560016 104.902) (end 88.814016 105.156) (width 0.508) (layer "B.Cu") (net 5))
 (segment (start 87.017551 104.902) (end 88.560016 104.902) (width 0.508) (layer "B.Cu") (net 5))
 (segment (start 226.822 141.478) (end 224.028 138.684) (width 0.508) (layer "B.Cu") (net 5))
 (segment (start 215.9 138.684) (end 215.392 138.684) (width 0.508) (layer "B.Cu") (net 5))
 (segment (start 224.028 138.684) (end 215.9 138.684) (width 0.508) (layer "B.Cu") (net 5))
 (segment (start 85.264 103.148449) (end 87.017551 104.902) (width 0.508) (layer "B.Cu") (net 5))
 (segment (start 88.814016 105.156) (end 211.328 140.97) (width 0.508) (layer "B.Cu") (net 5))
 (segment (start 85.264 96.52) (end 85.264 103.148449) (width 0.508) (layer "B.Cu") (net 5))
 (segment (start 213.868 139.954) (end 86.614 102.87) (width 0.762) (layer "B.Cu") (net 6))
 (segment (start 86.514 96.52) (end 86.614 96.62) (width 0.762) (layer "B.Cu") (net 6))
 (segment (start 214.122 140.208) (end 213.868 139.954) (width 0.762) (layer "B.Cu") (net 6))
 (segment (start 214.122 141.478) (end 214.122 140.208) (width 0.762) (layer "B.Cu") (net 6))
 (segment (start 86.614 96.62) (end 86.614 102.87) (width 0.762) (layer "B.Cu") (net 6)))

